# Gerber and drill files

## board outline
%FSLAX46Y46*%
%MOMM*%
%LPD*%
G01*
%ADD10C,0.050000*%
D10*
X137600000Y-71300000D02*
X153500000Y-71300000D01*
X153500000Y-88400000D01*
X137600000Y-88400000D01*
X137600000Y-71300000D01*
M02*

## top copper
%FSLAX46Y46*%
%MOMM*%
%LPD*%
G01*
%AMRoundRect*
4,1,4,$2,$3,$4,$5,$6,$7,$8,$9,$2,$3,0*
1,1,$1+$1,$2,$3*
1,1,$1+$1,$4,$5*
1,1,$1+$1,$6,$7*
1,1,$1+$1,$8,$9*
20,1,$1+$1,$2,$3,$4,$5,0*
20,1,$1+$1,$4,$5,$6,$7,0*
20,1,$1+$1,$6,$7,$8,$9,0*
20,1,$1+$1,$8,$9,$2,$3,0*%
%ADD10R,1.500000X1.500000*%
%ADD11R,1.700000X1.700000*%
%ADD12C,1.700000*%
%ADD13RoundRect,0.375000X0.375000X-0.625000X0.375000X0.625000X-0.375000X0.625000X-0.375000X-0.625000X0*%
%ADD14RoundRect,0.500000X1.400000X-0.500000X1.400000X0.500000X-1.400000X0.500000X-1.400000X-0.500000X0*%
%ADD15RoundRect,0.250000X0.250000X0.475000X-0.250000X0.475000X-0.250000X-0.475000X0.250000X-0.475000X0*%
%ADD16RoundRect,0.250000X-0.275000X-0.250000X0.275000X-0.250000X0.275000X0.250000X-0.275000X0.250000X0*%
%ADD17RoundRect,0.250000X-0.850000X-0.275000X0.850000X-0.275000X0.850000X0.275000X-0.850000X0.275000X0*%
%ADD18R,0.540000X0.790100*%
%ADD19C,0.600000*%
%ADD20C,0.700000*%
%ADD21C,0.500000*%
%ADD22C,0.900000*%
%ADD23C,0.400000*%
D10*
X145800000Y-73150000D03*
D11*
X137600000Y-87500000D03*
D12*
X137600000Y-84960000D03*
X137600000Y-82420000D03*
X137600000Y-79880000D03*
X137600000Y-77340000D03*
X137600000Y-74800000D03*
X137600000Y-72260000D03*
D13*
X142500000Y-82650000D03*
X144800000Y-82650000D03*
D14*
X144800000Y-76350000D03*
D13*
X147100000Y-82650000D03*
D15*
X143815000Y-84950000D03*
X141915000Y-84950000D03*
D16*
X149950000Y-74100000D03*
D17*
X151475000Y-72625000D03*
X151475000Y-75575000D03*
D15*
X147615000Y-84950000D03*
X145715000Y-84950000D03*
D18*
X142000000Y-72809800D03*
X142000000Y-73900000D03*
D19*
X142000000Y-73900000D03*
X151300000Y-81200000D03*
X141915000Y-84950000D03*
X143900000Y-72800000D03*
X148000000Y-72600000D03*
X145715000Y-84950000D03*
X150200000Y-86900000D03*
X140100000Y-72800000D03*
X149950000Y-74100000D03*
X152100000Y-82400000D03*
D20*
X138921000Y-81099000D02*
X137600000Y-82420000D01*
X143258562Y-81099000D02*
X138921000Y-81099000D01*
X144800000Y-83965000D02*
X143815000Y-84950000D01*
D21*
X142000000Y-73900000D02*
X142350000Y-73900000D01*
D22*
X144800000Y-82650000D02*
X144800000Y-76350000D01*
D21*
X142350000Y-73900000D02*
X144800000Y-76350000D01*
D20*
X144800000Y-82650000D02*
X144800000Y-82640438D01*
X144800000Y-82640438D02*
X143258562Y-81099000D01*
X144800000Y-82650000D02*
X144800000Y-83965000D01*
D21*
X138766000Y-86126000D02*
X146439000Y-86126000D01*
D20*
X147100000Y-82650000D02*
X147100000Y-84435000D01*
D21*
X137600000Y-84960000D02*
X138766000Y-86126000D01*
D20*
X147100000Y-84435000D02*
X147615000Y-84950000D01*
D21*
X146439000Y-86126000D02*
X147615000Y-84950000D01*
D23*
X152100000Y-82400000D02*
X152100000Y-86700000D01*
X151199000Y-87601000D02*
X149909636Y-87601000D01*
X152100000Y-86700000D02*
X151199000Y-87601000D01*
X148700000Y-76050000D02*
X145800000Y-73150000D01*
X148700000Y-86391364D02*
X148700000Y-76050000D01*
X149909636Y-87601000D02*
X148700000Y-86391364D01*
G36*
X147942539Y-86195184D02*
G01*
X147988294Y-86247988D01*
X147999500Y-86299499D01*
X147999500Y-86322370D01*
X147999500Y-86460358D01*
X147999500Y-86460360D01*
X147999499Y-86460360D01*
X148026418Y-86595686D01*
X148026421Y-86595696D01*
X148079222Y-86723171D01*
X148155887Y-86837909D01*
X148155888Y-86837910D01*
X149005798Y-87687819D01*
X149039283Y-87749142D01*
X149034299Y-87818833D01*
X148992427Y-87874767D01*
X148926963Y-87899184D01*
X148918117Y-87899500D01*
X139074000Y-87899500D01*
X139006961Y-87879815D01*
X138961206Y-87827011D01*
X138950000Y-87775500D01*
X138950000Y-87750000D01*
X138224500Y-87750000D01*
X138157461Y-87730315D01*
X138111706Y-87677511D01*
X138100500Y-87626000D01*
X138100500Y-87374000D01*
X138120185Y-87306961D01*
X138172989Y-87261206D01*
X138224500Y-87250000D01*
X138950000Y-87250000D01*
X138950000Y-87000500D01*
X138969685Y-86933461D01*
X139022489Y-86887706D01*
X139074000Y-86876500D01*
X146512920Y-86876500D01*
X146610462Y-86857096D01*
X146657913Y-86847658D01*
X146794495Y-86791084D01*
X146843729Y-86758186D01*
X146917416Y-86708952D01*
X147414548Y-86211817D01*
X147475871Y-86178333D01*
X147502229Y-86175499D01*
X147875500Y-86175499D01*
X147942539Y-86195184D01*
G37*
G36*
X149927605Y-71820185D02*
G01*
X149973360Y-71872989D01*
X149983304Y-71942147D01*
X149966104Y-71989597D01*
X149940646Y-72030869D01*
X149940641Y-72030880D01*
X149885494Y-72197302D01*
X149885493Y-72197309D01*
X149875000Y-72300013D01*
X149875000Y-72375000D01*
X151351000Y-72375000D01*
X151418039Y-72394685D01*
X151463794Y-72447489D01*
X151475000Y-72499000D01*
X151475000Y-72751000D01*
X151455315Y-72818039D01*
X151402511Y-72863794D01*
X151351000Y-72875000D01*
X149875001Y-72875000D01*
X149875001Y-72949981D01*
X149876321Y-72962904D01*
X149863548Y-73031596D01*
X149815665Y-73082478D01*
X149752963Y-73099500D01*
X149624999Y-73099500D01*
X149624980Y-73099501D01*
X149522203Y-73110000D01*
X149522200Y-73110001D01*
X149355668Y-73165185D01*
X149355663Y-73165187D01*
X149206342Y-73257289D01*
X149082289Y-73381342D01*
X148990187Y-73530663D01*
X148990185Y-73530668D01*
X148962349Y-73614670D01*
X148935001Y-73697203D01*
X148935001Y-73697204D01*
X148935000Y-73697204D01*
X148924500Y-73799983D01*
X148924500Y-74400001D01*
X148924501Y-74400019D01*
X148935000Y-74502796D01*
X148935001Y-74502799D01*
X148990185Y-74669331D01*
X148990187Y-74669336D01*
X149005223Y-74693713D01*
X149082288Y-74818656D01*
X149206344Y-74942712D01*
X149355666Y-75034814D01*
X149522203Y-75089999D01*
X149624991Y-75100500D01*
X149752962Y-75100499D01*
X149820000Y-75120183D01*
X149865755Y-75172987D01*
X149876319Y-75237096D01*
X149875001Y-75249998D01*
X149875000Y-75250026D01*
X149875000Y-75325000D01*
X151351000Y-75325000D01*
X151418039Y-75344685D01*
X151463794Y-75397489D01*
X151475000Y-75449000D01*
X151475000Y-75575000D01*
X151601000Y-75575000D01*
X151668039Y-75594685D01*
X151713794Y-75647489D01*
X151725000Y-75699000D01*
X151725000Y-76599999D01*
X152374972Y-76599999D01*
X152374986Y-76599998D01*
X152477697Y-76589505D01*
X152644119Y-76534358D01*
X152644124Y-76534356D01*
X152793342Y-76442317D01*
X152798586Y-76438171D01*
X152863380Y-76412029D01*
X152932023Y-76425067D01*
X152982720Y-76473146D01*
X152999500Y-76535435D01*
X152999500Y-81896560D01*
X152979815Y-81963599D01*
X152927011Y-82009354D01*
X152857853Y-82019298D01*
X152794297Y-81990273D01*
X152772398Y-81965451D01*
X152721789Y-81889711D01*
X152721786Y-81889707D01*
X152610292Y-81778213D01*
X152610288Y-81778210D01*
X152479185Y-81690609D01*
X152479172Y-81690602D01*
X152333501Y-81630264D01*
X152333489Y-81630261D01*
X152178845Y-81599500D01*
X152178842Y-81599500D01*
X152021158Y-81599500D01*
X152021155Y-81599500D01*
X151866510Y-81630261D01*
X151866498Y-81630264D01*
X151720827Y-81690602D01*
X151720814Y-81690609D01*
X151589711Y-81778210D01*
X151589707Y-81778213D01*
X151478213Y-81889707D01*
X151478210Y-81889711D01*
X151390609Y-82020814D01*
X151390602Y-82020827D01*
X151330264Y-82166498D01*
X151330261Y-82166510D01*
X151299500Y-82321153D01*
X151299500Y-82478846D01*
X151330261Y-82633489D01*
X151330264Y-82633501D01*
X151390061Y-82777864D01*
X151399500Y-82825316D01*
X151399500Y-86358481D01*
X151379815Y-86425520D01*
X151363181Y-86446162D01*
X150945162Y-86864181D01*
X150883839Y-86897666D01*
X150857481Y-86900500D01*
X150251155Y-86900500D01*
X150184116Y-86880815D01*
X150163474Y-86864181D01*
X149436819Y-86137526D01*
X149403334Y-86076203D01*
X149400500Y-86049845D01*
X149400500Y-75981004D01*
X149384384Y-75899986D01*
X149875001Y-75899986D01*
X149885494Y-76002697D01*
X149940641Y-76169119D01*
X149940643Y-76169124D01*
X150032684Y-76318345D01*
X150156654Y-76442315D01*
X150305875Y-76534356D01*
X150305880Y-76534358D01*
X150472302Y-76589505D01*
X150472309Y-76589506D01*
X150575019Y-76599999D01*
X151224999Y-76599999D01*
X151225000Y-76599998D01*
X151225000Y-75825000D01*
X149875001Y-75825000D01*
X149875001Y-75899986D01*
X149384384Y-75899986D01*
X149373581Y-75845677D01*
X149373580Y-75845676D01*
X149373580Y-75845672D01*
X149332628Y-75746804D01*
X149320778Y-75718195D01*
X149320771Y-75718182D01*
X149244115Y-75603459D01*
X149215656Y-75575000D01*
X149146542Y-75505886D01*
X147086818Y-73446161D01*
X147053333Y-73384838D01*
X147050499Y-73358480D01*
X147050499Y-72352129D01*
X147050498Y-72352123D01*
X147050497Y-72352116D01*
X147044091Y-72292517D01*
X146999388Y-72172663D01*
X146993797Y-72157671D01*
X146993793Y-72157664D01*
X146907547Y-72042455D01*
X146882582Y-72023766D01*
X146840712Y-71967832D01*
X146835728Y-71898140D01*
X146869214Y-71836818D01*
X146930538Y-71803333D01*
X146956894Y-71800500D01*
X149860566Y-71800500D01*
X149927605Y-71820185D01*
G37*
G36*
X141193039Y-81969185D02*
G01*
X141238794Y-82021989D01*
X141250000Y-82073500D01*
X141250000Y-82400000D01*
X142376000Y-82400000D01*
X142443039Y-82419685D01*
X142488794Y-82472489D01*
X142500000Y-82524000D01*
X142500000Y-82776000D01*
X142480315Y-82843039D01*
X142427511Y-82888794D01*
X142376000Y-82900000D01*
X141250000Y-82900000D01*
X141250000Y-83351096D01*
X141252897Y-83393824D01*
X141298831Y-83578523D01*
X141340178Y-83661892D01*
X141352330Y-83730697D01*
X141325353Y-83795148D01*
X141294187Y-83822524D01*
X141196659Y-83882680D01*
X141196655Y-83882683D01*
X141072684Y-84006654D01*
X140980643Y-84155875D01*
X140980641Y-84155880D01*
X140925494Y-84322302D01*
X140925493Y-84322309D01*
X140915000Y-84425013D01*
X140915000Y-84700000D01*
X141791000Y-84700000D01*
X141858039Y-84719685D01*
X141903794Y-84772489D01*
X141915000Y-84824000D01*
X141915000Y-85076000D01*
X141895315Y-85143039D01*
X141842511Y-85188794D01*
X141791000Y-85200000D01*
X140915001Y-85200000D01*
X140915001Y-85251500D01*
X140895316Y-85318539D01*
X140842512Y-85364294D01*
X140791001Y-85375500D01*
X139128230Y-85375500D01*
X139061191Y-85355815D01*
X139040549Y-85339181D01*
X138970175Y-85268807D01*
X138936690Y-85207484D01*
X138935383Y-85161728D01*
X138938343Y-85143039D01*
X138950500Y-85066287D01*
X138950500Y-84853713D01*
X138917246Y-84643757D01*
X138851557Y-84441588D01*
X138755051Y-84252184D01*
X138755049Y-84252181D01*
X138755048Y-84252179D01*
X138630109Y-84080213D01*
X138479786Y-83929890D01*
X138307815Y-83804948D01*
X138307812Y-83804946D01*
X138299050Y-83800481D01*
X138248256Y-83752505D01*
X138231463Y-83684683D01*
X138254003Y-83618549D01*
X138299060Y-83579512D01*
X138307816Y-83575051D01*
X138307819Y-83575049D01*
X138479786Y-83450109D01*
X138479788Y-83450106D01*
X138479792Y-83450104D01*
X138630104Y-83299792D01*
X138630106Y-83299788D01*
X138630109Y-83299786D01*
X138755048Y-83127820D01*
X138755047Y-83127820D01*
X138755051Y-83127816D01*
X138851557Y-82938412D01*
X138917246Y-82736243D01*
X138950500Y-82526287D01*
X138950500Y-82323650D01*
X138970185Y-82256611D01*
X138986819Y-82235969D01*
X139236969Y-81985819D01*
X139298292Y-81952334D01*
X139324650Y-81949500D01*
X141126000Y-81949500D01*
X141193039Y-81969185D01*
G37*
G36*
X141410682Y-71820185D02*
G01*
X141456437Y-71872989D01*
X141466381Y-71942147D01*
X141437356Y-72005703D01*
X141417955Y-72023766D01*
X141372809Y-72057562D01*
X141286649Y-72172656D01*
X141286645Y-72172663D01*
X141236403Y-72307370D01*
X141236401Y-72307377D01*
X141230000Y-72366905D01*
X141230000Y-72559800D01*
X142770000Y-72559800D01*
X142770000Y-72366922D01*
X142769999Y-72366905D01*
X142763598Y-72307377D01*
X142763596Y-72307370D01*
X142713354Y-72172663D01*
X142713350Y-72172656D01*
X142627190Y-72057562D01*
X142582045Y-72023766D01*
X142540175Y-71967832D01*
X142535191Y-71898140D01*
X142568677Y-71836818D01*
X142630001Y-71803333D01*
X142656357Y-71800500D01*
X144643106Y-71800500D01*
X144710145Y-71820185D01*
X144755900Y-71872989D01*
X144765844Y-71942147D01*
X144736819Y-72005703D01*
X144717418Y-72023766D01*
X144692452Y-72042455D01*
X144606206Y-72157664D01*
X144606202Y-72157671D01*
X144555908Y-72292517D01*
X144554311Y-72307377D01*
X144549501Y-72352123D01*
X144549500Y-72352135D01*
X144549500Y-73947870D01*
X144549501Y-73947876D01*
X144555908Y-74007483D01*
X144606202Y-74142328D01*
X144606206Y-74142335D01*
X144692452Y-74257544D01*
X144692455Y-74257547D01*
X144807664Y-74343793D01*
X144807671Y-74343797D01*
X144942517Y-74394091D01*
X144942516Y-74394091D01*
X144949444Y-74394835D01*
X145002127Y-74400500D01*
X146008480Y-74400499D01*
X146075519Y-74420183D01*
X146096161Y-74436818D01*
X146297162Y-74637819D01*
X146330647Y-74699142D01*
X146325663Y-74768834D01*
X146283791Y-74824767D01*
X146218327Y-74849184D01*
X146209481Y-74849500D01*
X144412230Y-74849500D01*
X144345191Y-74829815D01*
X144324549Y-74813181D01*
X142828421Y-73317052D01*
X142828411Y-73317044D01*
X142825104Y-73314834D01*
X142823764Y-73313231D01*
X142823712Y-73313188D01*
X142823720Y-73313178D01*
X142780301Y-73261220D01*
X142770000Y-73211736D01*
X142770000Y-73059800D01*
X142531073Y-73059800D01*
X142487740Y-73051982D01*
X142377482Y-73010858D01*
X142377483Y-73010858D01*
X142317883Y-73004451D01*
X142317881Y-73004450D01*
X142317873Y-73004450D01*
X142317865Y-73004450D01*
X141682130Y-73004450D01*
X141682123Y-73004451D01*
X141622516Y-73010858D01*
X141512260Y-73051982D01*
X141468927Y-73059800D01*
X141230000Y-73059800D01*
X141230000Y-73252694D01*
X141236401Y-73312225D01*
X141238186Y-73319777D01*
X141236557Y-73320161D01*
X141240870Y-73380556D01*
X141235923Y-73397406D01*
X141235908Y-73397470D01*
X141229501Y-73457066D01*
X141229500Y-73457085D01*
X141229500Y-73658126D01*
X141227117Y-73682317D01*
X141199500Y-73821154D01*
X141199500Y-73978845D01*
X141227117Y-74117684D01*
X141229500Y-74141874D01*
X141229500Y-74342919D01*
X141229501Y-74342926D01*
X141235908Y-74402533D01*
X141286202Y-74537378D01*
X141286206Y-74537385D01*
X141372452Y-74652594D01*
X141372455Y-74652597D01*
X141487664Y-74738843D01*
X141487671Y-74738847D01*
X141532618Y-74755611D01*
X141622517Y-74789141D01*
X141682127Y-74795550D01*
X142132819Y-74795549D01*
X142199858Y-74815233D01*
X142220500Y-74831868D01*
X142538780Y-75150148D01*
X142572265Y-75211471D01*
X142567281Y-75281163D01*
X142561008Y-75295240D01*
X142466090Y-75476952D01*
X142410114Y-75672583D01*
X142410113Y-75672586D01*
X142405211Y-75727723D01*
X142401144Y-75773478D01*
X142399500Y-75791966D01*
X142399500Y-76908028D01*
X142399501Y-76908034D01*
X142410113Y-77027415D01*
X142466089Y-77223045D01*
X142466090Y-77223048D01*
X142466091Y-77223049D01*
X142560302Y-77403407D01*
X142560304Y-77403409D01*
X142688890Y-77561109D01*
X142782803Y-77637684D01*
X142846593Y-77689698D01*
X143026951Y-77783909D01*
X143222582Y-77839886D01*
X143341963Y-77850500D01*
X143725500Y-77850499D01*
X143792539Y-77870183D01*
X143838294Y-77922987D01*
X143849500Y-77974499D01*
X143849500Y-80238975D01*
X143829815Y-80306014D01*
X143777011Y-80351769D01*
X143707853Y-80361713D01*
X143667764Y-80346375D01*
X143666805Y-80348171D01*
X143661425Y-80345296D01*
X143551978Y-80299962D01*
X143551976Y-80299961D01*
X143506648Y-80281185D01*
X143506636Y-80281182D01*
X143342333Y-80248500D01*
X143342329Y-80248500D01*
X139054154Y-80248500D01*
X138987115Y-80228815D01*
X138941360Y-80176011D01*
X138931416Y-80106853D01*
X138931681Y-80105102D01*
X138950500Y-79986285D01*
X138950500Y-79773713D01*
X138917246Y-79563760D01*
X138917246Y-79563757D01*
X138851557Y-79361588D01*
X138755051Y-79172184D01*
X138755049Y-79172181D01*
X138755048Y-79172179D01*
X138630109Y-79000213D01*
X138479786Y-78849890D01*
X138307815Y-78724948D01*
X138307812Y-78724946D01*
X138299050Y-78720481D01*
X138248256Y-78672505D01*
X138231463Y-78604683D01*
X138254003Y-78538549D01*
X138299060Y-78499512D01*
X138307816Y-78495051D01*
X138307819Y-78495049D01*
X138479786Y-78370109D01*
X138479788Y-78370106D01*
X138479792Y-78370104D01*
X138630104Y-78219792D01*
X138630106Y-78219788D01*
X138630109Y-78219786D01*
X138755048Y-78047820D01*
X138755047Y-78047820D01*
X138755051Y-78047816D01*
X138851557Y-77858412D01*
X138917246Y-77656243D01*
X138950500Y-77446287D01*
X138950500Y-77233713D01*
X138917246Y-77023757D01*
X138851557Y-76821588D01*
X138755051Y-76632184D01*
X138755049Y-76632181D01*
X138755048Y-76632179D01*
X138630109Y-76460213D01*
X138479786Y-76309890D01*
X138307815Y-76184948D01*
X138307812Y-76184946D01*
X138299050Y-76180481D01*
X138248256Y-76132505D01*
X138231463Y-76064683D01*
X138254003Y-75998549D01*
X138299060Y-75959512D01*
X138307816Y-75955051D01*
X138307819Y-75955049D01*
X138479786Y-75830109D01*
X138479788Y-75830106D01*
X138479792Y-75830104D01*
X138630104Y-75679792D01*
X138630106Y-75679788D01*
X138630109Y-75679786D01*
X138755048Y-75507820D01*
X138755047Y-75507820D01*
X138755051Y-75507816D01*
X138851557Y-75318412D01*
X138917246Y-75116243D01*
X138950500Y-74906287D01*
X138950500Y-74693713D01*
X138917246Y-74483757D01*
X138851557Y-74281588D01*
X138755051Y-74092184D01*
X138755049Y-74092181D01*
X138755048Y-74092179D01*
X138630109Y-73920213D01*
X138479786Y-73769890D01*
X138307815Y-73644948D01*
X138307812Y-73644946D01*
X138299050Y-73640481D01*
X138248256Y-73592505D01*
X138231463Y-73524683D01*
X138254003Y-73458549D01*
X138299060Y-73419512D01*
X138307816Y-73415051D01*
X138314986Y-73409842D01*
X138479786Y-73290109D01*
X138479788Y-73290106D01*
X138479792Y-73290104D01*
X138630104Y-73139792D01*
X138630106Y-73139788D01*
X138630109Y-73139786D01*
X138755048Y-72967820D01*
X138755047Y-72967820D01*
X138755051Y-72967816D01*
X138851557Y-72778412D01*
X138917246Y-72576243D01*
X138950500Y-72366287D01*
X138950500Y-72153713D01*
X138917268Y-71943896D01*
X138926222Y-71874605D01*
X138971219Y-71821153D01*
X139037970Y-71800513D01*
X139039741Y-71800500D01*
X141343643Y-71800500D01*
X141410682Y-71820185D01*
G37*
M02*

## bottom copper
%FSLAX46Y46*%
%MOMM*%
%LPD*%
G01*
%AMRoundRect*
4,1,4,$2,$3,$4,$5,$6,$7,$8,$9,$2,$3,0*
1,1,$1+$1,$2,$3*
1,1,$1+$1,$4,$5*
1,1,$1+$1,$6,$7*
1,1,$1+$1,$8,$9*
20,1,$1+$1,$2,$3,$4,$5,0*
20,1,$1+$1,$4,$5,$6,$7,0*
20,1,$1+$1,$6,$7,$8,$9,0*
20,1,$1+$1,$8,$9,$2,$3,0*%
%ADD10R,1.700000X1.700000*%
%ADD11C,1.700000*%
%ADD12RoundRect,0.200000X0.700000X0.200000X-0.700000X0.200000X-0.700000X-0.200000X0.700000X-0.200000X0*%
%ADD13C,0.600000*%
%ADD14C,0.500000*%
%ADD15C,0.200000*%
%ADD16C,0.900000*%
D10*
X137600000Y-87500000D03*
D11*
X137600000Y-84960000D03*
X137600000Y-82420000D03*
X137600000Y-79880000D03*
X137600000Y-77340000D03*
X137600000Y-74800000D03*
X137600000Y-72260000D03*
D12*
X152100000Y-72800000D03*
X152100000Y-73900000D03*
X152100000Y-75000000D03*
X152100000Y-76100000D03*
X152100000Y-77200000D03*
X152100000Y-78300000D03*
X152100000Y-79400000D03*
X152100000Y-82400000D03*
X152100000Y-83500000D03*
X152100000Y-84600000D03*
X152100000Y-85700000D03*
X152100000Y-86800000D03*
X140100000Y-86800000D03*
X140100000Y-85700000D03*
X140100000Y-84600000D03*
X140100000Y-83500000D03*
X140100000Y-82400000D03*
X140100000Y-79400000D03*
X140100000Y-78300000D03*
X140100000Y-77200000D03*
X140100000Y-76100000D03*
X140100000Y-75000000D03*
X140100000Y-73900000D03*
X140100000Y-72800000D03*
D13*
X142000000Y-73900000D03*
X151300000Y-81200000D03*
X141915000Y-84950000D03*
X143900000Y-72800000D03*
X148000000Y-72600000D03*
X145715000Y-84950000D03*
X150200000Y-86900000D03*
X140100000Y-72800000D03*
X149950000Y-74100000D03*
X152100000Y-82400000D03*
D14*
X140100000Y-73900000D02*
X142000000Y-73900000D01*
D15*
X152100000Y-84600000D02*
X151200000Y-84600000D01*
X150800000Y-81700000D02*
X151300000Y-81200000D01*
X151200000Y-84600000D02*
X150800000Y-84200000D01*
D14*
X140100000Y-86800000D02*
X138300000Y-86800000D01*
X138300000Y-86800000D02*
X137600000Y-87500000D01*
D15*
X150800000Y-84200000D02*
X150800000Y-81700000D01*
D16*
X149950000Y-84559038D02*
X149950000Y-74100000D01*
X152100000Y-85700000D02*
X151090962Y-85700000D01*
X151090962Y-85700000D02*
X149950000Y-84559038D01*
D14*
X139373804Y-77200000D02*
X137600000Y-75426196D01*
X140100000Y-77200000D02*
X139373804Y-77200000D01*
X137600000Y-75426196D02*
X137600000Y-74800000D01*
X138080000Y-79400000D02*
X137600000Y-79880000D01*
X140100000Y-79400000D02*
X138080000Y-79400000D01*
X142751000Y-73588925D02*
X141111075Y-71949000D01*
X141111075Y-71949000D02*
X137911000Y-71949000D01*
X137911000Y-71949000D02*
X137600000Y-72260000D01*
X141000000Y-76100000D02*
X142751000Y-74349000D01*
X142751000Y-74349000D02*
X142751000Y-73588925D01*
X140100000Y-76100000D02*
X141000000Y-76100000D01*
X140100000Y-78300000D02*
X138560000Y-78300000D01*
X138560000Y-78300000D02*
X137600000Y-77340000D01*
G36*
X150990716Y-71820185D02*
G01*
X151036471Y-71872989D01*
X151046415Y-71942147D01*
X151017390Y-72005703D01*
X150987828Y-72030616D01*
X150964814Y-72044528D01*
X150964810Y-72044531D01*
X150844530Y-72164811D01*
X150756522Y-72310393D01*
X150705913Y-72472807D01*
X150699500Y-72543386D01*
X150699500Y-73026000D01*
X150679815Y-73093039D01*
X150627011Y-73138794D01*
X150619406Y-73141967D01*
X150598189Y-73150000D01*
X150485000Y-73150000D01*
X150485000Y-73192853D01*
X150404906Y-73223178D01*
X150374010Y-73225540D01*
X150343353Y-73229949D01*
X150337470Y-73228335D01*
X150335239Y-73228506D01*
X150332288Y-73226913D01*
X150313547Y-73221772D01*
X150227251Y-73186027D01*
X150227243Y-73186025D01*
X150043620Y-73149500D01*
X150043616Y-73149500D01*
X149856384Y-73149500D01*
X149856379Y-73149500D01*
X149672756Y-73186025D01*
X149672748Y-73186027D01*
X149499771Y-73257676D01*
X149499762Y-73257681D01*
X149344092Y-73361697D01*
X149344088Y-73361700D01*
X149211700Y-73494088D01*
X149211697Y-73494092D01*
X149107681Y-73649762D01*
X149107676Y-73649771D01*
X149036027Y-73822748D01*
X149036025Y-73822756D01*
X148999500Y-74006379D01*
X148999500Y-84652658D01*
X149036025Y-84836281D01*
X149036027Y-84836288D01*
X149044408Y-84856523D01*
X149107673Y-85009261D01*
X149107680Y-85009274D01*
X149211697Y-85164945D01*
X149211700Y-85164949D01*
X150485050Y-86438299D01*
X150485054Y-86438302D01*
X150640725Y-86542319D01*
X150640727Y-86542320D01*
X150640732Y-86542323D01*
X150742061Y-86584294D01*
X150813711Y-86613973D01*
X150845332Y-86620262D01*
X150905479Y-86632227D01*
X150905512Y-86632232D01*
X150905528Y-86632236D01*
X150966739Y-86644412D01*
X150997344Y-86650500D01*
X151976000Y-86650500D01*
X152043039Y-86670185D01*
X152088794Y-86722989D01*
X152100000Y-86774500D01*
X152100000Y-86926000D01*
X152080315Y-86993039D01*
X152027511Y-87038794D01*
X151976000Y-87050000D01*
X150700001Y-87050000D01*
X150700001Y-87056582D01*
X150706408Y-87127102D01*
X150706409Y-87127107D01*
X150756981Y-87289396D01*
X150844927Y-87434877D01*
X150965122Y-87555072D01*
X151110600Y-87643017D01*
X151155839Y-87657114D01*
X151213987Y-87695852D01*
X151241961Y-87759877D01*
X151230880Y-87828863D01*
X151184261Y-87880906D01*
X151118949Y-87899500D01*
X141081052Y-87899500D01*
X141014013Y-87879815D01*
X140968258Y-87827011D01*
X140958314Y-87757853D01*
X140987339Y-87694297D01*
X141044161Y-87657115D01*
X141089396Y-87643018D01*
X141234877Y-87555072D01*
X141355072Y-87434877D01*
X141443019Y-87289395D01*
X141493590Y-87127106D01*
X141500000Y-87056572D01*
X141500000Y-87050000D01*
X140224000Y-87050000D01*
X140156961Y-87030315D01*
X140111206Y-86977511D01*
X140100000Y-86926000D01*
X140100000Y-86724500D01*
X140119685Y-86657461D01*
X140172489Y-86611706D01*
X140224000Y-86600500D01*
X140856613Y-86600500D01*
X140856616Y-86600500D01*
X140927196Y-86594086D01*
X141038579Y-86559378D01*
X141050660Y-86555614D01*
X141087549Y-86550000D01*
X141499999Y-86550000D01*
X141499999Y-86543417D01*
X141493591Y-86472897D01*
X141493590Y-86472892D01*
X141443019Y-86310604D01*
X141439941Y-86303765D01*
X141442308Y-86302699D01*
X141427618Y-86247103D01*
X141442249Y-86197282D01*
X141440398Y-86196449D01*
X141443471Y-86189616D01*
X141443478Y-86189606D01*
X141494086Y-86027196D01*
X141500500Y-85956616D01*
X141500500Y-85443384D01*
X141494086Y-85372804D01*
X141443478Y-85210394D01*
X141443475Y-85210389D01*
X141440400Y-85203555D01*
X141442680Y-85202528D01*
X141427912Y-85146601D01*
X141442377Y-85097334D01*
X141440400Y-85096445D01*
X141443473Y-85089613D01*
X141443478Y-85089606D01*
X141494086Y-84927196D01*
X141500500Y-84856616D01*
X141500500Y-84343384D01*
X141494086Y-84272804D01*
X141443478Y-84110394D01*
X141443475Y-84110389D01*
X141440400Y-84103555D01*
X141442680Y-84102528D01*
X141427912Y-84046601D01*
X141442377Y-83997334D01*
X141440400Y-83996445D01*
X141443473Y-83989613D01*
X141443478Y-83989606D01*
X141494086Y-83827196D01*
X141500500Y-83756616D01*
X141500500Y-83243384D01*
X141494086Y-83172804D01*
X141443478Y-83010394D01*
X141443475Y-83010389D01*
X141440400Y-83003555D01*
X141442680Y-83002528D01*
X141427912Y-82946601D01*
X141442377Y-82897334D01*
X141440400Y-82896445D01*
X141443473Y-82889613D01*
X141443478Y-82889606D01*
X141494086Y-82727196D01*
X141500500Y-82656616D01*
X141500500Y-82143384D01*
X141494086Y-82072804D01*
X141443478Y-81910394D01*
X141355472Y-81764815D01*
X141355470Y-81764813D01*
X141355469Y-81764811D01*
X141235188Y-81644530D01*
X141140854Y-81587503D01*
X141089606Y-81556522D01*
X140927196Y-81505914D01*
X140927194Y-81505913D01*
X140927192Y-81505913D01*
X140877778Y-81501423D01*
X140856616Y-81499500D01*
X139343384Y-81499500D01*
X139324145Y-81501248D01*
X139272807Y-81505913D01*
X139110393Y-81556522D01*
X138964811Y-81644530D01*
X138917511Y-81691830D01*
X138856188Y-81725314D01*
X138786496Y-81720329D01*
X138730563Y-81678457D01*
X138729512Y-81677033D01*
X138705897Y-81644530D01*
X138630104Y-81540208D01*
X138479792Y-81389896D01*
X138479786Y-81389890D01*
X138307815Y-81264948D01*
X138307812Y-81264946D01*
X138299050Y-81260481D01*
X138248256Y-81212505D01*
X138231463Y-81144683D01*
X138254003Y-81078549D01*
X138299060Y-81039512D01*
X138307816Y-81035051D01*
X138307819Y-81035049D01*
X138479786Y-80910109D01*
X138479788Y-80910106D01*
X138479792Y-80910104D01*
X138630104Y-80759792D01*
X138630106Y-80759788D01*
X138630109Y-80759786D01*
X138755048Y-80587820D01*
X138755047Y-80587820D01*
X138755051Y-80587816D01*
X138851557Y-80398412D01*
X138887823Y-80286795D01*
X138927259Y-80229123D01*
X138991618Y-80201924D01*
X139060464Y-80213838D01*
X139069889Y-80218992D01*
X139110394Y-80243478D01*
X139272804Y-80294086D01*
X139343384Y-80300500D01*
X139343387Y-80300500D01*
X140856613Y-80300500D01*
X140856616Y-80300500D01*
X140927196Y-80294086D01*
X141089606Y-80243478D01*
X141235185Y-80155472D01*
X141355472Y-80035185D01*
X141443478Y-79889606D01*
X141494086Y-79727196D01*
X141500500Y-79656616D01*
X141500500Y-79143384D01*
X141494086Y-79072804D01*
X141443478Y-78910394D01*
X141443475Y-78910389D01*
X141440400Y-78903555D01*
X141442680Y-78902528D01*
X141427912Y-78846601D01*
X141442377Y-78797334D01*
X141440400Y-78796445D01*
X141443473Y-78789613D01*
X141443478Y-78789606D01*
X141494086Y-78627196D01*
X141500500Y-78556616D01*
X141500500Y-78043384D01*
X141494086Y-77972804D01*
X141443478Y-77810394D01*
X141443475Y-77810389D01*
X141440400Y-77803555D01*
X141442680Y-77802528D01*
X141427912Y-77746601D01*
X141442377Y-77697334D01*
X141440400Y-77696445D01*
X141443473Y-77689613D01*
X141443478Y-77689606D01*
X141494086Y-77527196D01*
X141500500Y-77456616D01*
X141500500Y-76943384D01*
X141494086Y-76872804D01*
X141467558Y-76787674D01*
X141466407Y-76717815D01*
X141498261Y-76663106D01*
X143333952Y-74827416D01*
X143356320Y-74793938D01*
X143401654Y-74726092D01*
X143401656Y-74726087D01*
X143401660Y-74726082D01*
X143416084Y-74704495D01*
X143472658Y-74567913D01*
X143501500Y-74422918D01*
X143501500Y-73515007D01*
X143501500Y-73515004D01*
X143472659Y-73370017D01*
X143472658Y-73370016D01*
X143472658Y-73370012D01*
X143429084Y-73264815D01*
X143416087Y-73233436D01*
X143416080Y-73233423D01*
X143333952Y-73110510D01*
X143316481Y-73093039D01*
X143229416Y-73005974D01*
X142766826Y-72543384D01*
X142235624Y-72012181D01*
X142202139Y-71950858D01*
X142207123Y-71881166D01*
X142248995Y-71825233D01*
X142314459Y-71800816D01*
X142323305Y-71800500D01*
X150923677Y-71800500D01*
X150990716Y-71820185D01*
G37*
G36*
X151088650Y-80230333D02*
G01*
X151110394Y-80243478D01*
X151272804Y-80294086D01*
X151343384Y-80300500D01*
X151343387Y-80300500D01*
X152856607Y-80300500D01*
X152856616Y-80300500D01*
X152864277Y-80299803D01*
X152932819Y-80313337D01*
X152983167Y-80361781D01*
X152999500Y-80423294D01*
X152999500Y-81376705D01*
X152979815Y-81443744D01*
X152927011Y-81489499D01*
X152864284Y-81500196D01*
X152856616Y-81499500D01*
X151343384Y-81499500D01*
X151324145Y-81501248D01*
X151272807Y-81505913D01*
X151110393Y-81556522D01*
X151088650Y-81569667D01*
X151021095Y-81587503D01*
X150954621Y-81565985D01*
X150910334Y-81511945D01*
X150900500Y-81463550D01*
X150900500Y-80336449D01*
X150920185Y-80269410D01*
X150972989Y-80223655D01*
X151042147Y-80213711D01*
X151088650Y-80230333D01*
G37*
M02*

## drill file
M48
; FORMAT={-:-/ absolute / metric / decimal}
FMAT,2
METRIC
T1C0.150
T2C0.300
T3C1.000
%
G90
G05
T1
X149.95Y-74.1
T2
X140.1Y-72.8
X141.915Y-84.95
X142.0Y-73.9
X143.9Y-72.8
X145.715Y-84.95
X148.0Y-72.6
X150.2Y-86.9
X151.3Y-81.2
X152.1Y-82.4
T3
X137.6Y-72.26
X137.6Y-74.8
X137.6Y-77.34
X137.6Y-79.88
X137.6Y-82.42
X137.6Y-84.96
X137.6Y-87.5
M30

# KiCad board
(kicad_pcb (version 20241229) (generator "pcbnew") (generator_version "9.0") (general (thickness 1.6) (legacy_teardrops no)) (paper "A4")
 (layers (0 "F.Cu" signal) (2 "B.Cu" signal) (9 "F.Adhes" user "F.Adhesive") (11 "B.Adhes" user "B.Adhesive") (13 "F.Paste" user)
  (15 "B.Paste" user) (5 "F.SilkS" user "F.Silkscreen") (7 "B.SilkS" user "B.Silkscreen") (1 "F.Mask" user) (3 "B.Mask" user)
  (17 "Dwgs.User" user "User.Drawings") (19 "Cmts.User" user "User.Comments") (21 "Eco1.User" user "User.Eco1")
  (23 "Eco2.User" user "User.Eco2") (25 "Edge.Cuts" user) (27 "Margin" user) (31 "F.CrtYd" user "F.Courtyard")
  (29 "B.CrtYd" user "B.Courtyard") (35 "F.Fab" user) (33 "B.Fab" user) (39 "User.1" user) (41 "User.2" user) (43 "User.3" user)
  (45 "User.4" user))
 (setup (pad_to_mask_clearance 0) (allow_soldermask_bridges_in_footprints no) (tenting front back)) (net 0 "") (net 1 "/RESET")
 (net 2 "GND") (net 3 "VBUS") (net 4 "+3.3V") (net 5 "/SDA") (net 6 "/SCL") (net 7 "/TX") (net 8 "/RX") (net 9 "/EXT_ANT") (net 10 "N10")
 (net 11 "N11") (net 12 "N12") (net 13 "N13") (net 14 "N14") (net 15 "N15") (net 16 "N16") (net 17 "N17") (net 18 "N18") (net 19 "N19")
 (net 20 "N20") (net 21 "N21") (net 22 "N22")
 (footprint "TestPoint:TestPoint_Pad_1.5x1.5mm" (layer "F.Cu") (at 145.8 73.15)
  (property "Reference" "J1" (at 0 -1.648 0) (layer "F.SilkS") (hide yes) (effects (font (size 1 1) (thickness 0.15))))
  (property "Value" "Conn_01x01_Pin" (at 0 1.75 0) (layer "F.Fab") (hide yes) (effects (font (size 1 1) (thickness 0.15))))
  (pad "1" smd rect (at 0 0) (size 1.5 1.5) (layers "F.Cu" "F.Mask") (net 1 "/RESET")))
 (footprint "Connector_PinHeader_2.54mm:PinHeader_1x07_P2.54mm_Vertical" (layer "F.Cu") (at 137.6 87.5 180)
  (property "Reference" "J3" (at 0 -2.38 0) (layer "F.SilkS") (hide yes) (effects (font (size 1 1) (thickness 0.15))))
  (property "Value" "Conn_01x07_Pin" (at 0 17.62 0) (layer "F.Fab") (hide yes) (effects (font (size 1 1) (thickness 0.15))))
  (pad "1" thru_hole rect (at 0 0 180) (size 1.7 1.7) (drill 1) (layers "*.Cu" "*.Mask") (remove_unused_layers no) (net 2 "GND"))
  (pad "2" thru_hole circle (at 0 2.54 180) (size 1.7 1.7) (drill 1) (layers "*.Cu" "*.Mask") (remove_unused_layers no) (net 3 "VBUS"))
  (pad "3" thru_hole circle (at 0 5.08 180) (size 1.7 1.7) (drill 1) (layers "*.Cu" "*.Mask") (remove_unused_layers no) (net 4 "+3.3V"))
  (pad "4" thru_hole circle (at 0 7.62 180) (size 1.7 1.7) (drill 1) (layers "*.Cu" "*.Mask") (remove_unused_layers no) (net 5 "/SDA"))
  (pad "5" thru_hole circle (at 0 10.16 180) (size 1.7 1.7) (drill 1) (layers "*.Cu" "*.Mask") (remove_unused_layers no) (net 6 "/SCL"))
  (pad "6" thru_hole circle (at 0 12.7 180) (size 1.7 1.7) (drill 1) (layers "*.Cu" "*.Mask") (remove_unused_layers no) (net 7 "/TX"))
  (pad "7" thru_hole circle (at 0 15.24 180) (size 1.7 1.7) (drill 1) (layers "*.Cu" "*.Mask") (remove_unused_layers no) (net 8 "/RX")))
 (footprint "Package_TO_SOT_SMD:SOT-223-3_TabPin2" (layer "F.Cu") (at 144.8 79.5 90)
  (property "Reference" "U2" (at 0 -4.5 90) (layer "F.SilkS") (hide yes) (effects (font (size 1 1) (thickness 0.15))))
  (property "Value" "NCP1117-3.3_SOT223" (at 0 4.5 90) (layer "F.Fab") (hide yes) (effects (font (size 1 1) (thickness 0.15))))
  (pad "1" smd roundrect (at -3.15 -2.3 90) (size 2 1.5) (layers "F.Cu" "F.Mask" "F.Paste") (roundrect_rratio 0.25) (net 2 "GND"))
  (pad "2" smd roundrect (at -3.15 0 90) (size 2 1.5) (layers "F.Cu" "F.Mask" "F.Paste") (roundrect_rratio 0.25) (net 4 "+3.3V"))
  (pad "2" smd roundrect (at 3.15 0 90) (size 2 3.8) (layers "F.Cu" "F.Mask" "F.Paste") (roundrect_rratio 0.25) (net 4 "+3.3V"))
  (pad "3" smd roundrect (at -3.15 2.3 90) (size 2 1.5) (layers "F.Cu" "F.Mask" "F.Paste") (roundrect_rratio 0.25) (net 3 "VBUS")))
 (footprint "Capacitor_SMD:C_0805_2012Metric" (layer "F.Cu") (at 142.865 84.95 180)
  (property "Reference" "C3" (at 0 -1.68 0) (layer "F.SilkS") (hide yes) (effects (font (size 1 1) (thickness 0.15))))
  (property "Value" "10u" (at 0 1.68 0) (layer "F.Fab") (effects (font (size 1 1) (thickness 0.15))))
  (pad "1" smd roundrect (at -0.95 0 180) (size 1 1.45) (layers "F.Cu" "F.Mask" "F.Paste") (roundrect_rratio 0.25) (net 4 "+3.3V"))
  (pad "2" smd roundrect (at 0.95 0 180) (size 1 1.45) (layers "F.Cu" "F.Mask" "F.Paste") (roundrect_rratio 0.25) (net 2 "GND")))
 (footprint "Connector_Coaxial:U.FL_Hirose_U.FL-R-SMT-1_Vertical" (layer "F.Cu") (at 151 74.1)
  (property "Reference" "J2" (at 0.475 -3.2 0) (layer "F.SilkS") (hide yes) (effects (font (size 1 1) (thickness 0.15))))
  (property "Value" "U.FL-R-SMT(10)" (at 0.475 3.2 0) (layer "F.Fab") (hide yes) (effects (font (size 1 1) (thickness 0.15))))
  (pad "1" smd roundrect (at -1.05 0) (size 1.05 1) (layers "F.Cu" "F.Mask" "F.Paste") (roundrect_rratio 0.25) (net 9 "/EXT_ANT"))
  (pad "2" smd roundrect (at 0.475 -1.475) (size 2.2 1.05) (layers "F.Cu" "F.Mask" "F.Paste") (roundrect_rratio 0.2380952381) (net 2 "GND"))
  (pad "2" smd roundrect (at 0.475 1.475) (size 2.2 1.05) (layers "F.Cu" "F.Mask" "F.Paste") (roundrect_rratio 0.2380952381) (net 2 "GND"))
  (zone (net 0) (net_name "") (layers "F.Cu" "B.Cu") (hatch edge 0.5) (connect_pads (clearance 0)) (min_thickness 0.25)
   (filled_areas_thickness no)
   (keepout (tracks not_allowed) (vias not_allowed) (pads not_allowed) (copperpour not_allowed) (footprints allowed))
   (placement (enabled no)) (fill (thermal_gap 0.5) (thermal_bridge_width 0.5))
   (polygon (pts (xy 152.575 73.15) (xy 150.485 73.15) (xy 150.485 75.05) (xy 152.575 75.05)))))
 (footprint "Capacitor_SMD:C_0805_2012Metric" (layer "F.Cu") (at 146.665 84.95 180)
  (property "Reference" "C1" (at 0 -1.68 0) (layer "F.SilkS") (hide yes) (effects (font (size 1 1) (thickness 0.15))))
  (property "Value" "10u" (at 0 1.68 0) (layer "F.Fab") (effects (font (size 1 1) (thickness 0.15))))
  (pad "1" smd roundrect (at -0.95 0 180) (size 1 1.45) (layers "F.Cu" "F.Mask" "F.Paste") (roundrect_rratio 0.25) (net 3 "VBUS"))
  (pad "2" smd roundrect (at 0.95 0 180) (size 1 1.45) (layers "F.Cu" "F.Mask" "F.Paste") (roundrect_rratio 0.25) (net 2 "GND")))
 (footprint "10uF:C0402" (layer "F.Cu") (at 142 73.3549 -90)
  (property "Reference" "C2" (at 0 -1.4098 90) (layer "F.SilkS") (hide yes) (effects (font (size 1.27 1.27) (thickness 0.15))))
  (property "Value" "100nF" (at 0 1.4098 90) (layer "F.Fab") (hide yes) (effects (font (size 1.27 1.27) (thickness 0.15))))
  (pad "1" smd rect (at -0.5451 0 270) (size 0.7901 0.54) (layers "F.Cu" "F.Mask" "F.Paste") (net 2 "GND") (solder_mask_margin 0.0508)
   (solder_paste_margin -100) (thermal_bridge_angle 0))
  (pad "2" smd rect (at 0.5451 0 270) (size 0.7901 0.54) (layers "F.Cu" "F.Mask" "F.Paste") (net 4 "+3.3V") (solder_mask_margin 0.0508)
   (solder_paste_margin -100) (thermal_bridge_angle 0))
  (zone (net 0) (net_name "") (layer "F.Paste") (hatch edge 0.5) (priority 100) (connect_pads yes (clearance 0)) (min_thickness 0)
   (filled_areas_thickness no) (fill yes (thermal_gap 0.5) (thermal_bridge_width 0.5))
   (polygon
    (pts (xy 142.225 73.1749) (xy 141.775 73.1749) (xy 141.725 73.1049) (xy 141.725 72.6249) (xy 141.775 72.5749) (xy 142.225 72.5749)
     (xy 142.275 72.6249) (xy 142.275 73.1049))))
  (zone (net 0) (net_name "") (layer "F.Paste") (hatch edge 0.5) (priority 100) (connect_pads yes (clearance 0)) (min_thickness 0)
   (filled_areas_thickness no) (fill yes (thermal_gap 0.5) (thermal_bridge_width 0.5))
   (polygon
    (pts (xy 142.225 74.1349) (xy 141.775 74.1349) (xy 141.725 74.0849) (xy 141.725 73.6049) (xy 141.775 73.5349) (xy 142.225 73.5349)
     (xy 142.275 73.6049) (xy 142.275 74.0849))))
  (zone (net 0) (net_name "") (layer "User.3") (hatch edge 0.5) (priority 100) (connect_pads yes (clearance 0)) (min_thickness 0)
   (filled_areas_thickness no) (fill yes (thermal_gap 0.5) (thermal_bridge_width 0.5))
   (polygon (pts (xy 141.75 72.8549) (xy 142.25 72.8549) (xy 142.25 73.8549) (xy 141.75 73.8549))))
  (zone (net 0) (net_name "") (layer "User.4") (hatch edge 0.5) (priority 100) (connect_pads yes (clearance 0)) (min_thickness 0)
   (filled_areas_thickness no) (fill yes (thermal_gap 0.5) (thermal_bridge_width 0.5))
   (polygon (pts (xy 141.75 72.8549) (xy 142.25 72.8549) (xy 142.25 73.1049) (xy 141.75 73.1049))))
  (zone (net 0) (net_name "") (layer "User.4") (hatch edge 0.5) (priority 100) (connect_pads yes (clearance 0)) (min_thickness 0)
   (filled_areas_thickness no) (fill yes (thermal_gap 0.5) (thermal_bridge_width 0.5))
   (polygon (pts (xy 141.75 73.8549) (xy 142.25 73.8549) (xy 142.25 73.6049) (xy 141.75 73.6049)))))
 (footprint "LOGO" (layer "F.Cu") (at 150.6 78.6 -90)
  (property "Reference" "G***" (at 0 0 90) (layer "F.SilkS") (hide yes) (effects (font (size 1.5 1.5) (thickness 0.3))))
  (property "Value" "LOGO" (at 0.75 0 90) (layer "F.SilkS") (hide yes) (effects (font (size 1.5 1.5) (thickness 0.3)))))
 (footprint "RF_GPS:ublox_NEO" (layer "B.Cu") (at 146.1 79.8 180)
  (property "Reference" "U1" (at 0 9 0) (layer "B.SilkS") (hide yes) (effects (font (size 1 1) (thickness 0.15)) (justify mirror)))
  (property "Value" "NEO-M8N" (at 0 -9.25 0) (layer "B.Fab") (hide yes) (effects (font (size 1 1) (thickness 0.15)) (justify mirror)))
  (pad "1" smd roundrect (at -6 7 180) (size 1.8 0.8) (layers "B.Cu" "B.Mask" "B.Paste") (roundrect_rratio 0.25) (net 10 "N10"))
  (pad "2" smd roundrect (at -6 5.9 180) (size 1.8 0.8) (layers "B.Cu" "B.Mask" "B.Paste") (roundrect_rratio 0.25) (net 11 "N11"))
  (pad "3" smd roundrect (at -6 4.8 180) (size 1.8 0.8) (layers "B.Cu" "B.Mask" "B.Paste") (roundrect_rratio 0.25) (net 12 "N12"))
  (pad "4" smd roundrect (at -6 3.7 180) (size 1.8 0.8) (layers "B.Cu" "B.Mask" "B.Paste") (roundrect_rratio 0.25) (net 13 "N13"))
  (pad "5" smd roundrect (at -6 2.6 180) (size 1.8 0.8) (layers "B.Cu" "B.Mask" "B.Paste") (roundrect_rratio 0.25) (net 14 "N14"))
  (pad "6" smd roundrect (at -6 1.5 180) (size 1.8 0.8) (layers "B.Cu" "B.Mask" "B.Paste") (roundrect_rratio 0.25) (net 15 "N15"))
  (pad "7" smd roundrect (at -6 0.4 180) (size 1.8 0.8) (layers "B.Cu" "B.Mask" "B.Paste") (roundrect_rratio 0.25) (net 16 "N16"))
  (pad "8" smd roundrect (at -6 -2.6 180) (size 1.8 0.8) (layers "B.Cu" "B.Mask" "B.Paste") (roundrect_rratio 0.25) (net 1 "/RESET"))
  (pad "9" smd roundrect (at -6 -3.7 180) (size 1.8 0.8) (layers "B.Cu" "B.Mask" "B.Paste") (roundrect_rratio 0.25) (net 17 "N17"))
  (pad "10" smd roundrect (at -6 -4.8 180) (size 1.8 0.8) (layers "B.Cu" "B.Mask" "B.Paste") (roundrect_rratio 0.25) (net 2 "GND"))
  (pad "11" smd roundrect (at -6 -5.9 180) (size 1.8 0.8) (layers "B.Cu" "B.Mask" "B.Paste") (roundrect_rratio 0.25) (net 9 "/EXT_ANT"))
  (pad "12" smd roundrect (at -6 -7 180) (size 1.8 0.8) (layers "B.Cu" "B.Mask" "B.Paste") (roundrect_rratio 0.25) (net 2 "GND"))
  (pad "13" smd roundrect (at 6 -7 180) (size 1.8 0.8) (layers "B.Cu" "B.Mask" "B.Paste") (roundrect_rratio 0.25) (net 2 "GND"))
  (pad "14" smd roundrect (at 6 -5.9 180) (size 1.8 0.8) (layers "B.Cu" "B.Mask" "B.Paste") (roundrect_rratio 0.25) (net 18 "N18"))
  (pad "15" smd roundrect (at 6 -4.8 180) (size 1.8 0.8) (layers "B.Cu" "B.Mask" "B.Paste") (roundrect_rratio 0.25) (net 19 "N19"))
  (pad "16" smd roundrect (at 6 -3.7 180) (size 1.8 0.8) (layers "B.Cu" "B.Mask" "B.Paste") (roundrect_rratio 0.25) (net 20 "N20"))
  (pad "17" smd roundrect (at 6 -2.6 180) (size 1.8 0.8) (layers "B.Cu" "B.Mask" "B.Paste") (roundrect_rratio 0.25) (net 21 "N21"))
  (pad "18" smd roundrect (at 6 0.4 180) (size 1.8 0.8) (layers "B.Cu" "B.Mask" "B.Paste") (roundrect_rratio 0.25) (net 5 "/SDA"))
  (pad "19" smd roundrect (at 6 1.5 180) (size 1.8 0.8) (layers "B.Cu" "B.Mask" "B.Paste") (roundrect_rratio 0.25) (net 6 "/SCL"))
  (pad "20" smd roundrect (at 6 2.6 180) (size 1.8 0.8) (layers "B.Cu" "B.Mask" "B.Paste") (roundrect_rratio 0.25) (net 7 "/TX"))
  (pad "21" smd roundrect (at 6 3.7 180) (size 1.8 0.8) (layers "B.Cu" "B.Mask" "B.Paste") (roundrect_rratio 0.25) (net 8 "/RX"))
  (pad "22" smd roundrect (at 6 4.8 180) (size 1.8 0.8) (layers "B.Cu" "B.Mask" "B.Paste") (roundrect_rratio 0.25) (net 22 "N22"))
  (pad "23" smd roundrect (at 6 5.9 180) (size 1.8 0.8) (layers "B.Cu" "B.Mask" "B.Paste") (roundrect_rratio 0.25) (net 4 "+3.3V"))
  (pad "24" smd roundrect (at 6 7 180) (size 1.8 0.8) (layers "B.Cu" "B.Mask" "B.Paste") (roundrect_rratio 0.25) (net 2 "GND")))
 (gr_rect (start 137.6 71.3) (end 153.5 88.4) (stroke (width 0.05) (type default)) (fill no) (layer "Edge.Cuts"))
 (segment (start 138.921 81.099) (end 137.6 82.42) (width 0.7) (layer "F.Cu") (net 4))
 (segment (start 143.258562 81.099) (end 138.921 81.099) (width 0.7) (layer "F.Cu") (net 4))
 (segment (start 144.8 83.965) (end 143.815 84.95) (width 0.7) (layer "F.Cu") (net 4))
 (segment (start 142 73.9) (end 142.35 73.9) (width 0.5) (layer "F.Cu") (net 4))
 (segment (start 144.8 82.65) (end 144.8 76.35) (width 0.9) (layer "F.Cu") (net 4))
 (segment (start 142.35 73.9) (end 144.8 76.35) (width 0.5) (layer "F.Cu") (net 4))
 (segment (start 144.8 82.65) (end 144.8 82.640438) (width 0.7) (layer "F.Cu") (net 4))
 (segment (start 144.8 82.640438) (end 143.258562 81.099) (width 0.7) (layer "F.Cu") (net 4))
 (segment (start 144.8 82.65) (end 144.8 83.965) (width 0.7) (layer "F.Cu") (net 4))
 (via (at 142 73.9) (size 0.6) (drill 0.3) (layers "F.Cu" "B.Cu") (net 4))
 (segment (start 140.1 73.9) (end 142 73.9) (width 0.5) (layer "B.Cu") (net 4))
 (via (at 151.3 81.2) (size 0.6) (drill 0.3) (layers "F.Cu" "B.Cu") (free yes) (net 2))
 (via (at 141.915 84.95) (size 0.6) (drill 0.3) (layers "F.Cu" "B.Cu") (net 2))
 (via (at 143.9 72.8) (size 0.6) (drill 0.3) (layers "F.Cu" "B.Cu") (free yes) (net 2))
 (via (at 148 72.6) (size 0.6) (drill 0.3) (layers "F.Cu" "B.Cu") (free yes) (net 2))
 (via (at 145.715 84.95) (size 0.6) (drill 0.3) (layers "F.Cu" "B.Cu") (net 2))
 (via (at 150.2 86.9) (size 0.6) (drill 0.3) (layers "F.Cu" "B.Cu") (free yes) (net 2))
 (via (at 140.1 72.8) (size 0.6) (drill 0.3) (layers "F.Cu" "B.Cu") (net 2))
 (segment (start 152.1 84.6) (end 151.2 84.6) (width 0.2) (layer "B.Cu") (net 2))
 (segment (start 150.8 81.7) (end 151.3 81.2) (width 0.2) (layer "B.Cu") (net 2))
 (segment (start 151.2 84.6) (end 150.8 84.2) (width 0.2) (layer "B.Cu") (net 2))
 (segment (start 140.1 86.8) (end 138.3 86.8) (width 0.5) (layer "B.Cu") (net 2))
 (segment (start 138.3 86.8) (end 137.6 87.5) (width 0.5) (layer "B.Cu") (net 2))
 (segment (start 150.8 84.2) (end 150.8 81.7) (width 0.2) (layer "B.Cu") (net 2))
 (segment (start 138.766 86.126) (end 146.439 86.126) (width 0.5) (layer "F.Cu") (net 3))
 (segment (start 147.1 82.65) (end 147.1 84.435) (width 0.7) (layer "F.Cu") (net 3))
 (segment (start 137.6 84.96) (end 138.766 86.126) (width 0.5) (layer "F.Cu") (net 3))
 (segment (start 147.1 84.435) (end 147.615 84.95) (width 0.7) (layer "F.Cu") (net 3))
 (segment (start 146.439 86.126) (end 147.615 84.95) (width 0.5) (layer "F.Cu") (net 3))
 (via (at 149.95 74.1) (size 0.6) (drill 0.15) (layers "F.Cu" "B.Cu") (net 9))
 (segment (start 149.95 84.559038) (end 149.95 74.1) (width 0.9) (layer "B.Cu") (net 9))
 (segment (start 152.1 85.7) (end 151.090962 85.7) (width 0.9) (layer "B.Cu") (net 9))
 (segment (start 151.090962 85.7) (end 149.95 84.559038) (width 0.9) (layer "B.Cu") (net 9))
 (segment (start 139.373804 77.2) (end 137.6 75.426196) (width 0.5) (layer "B.Cu") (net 7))
 (segment (start 140.1 77.2) (end 139.373804 77.2) (width 0.5) (layer "B.Cu") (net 7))
 (segment (start 137.6 75.426196) (end 137.6 74.8) (width 0.5) (layer "B.Cu") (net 7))
 (segment (start 138.08 79.4) (end 137.6 79.88) (width 0.5) (layer "B.Cu") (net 5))
 (segment (start 140.1 79.4) (end 138.08 79.4) (width 0.5) (layer "B.Cu") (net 5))
 (segment (start 142.751 73.588925) (end 141.111075 71.949) (width 0.5) (layer "B.Cu") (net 8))
 (segment (start 141.111075 71.949) (end 137.911 71.949) (width 0.5) (layer "B.Cu") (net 8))
 (segment (start 137.911 71.949) (end 137.6 72.26) (width 0.5) (layer "B.Cu") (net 8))
 (segment (start 141 76.1) (end 142.751 74.349) (width 0.5) (layer "B.Cu") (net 8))
 (segment (start 142.751 74.349) (end 142.751 73.588925) (width 0.5) (layer "B.Cu") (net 8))
 (segment (start 140.1 76.1) (end 141 76.1) (width 0.5) (layer "B.Cu") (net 8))
 (segment (start 140.1 78.3) (end 138.56 78.3) (width 0.5) (layer "B.Cu") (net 6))
 (segment (start 138.56 78.3) (end 137.6 77.34) (width 0.5) (layer "B.Cu") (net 6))
 (segment (start 152.1 82.4) (end 152.1 86.7) (width 0.4) (layer "F.Cu") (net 1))
 (segment (start 151.199 87.601) (end 149.909636 87.601) (width 0.4) (layer "F.Cu") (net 1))
 (segment (start 152.1 86.7) (end 151.199 87.601) (width 0.4) (layer "F.Cu") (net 1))
 (segment (start 148.7 76.05) (end 145.8 73.15) (width 0.4) (layer "F.Cu") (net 1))
 (segment (start 148.7 86.391364) (end 148.7 76.05) (width 0.4) (layer "F.Cu") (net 1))
 (segment (start 149.909636 87.601) (end 148.7 86.391364) (width 0.4) (layer "F.Cu") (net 1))
 (via (at 152.1 82.4) (size 0.6) (drill 0.3) (layers "F.Cu" "B.Cu") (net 1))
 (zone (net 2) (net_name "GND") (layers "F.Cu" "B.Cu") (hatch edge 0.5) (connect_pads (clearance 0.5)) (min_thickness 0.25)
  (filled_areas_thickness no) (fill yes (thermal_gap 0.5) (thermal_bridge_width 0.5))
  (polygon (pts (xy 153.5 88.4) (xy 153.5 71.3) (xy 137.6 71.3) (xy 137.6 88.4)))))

